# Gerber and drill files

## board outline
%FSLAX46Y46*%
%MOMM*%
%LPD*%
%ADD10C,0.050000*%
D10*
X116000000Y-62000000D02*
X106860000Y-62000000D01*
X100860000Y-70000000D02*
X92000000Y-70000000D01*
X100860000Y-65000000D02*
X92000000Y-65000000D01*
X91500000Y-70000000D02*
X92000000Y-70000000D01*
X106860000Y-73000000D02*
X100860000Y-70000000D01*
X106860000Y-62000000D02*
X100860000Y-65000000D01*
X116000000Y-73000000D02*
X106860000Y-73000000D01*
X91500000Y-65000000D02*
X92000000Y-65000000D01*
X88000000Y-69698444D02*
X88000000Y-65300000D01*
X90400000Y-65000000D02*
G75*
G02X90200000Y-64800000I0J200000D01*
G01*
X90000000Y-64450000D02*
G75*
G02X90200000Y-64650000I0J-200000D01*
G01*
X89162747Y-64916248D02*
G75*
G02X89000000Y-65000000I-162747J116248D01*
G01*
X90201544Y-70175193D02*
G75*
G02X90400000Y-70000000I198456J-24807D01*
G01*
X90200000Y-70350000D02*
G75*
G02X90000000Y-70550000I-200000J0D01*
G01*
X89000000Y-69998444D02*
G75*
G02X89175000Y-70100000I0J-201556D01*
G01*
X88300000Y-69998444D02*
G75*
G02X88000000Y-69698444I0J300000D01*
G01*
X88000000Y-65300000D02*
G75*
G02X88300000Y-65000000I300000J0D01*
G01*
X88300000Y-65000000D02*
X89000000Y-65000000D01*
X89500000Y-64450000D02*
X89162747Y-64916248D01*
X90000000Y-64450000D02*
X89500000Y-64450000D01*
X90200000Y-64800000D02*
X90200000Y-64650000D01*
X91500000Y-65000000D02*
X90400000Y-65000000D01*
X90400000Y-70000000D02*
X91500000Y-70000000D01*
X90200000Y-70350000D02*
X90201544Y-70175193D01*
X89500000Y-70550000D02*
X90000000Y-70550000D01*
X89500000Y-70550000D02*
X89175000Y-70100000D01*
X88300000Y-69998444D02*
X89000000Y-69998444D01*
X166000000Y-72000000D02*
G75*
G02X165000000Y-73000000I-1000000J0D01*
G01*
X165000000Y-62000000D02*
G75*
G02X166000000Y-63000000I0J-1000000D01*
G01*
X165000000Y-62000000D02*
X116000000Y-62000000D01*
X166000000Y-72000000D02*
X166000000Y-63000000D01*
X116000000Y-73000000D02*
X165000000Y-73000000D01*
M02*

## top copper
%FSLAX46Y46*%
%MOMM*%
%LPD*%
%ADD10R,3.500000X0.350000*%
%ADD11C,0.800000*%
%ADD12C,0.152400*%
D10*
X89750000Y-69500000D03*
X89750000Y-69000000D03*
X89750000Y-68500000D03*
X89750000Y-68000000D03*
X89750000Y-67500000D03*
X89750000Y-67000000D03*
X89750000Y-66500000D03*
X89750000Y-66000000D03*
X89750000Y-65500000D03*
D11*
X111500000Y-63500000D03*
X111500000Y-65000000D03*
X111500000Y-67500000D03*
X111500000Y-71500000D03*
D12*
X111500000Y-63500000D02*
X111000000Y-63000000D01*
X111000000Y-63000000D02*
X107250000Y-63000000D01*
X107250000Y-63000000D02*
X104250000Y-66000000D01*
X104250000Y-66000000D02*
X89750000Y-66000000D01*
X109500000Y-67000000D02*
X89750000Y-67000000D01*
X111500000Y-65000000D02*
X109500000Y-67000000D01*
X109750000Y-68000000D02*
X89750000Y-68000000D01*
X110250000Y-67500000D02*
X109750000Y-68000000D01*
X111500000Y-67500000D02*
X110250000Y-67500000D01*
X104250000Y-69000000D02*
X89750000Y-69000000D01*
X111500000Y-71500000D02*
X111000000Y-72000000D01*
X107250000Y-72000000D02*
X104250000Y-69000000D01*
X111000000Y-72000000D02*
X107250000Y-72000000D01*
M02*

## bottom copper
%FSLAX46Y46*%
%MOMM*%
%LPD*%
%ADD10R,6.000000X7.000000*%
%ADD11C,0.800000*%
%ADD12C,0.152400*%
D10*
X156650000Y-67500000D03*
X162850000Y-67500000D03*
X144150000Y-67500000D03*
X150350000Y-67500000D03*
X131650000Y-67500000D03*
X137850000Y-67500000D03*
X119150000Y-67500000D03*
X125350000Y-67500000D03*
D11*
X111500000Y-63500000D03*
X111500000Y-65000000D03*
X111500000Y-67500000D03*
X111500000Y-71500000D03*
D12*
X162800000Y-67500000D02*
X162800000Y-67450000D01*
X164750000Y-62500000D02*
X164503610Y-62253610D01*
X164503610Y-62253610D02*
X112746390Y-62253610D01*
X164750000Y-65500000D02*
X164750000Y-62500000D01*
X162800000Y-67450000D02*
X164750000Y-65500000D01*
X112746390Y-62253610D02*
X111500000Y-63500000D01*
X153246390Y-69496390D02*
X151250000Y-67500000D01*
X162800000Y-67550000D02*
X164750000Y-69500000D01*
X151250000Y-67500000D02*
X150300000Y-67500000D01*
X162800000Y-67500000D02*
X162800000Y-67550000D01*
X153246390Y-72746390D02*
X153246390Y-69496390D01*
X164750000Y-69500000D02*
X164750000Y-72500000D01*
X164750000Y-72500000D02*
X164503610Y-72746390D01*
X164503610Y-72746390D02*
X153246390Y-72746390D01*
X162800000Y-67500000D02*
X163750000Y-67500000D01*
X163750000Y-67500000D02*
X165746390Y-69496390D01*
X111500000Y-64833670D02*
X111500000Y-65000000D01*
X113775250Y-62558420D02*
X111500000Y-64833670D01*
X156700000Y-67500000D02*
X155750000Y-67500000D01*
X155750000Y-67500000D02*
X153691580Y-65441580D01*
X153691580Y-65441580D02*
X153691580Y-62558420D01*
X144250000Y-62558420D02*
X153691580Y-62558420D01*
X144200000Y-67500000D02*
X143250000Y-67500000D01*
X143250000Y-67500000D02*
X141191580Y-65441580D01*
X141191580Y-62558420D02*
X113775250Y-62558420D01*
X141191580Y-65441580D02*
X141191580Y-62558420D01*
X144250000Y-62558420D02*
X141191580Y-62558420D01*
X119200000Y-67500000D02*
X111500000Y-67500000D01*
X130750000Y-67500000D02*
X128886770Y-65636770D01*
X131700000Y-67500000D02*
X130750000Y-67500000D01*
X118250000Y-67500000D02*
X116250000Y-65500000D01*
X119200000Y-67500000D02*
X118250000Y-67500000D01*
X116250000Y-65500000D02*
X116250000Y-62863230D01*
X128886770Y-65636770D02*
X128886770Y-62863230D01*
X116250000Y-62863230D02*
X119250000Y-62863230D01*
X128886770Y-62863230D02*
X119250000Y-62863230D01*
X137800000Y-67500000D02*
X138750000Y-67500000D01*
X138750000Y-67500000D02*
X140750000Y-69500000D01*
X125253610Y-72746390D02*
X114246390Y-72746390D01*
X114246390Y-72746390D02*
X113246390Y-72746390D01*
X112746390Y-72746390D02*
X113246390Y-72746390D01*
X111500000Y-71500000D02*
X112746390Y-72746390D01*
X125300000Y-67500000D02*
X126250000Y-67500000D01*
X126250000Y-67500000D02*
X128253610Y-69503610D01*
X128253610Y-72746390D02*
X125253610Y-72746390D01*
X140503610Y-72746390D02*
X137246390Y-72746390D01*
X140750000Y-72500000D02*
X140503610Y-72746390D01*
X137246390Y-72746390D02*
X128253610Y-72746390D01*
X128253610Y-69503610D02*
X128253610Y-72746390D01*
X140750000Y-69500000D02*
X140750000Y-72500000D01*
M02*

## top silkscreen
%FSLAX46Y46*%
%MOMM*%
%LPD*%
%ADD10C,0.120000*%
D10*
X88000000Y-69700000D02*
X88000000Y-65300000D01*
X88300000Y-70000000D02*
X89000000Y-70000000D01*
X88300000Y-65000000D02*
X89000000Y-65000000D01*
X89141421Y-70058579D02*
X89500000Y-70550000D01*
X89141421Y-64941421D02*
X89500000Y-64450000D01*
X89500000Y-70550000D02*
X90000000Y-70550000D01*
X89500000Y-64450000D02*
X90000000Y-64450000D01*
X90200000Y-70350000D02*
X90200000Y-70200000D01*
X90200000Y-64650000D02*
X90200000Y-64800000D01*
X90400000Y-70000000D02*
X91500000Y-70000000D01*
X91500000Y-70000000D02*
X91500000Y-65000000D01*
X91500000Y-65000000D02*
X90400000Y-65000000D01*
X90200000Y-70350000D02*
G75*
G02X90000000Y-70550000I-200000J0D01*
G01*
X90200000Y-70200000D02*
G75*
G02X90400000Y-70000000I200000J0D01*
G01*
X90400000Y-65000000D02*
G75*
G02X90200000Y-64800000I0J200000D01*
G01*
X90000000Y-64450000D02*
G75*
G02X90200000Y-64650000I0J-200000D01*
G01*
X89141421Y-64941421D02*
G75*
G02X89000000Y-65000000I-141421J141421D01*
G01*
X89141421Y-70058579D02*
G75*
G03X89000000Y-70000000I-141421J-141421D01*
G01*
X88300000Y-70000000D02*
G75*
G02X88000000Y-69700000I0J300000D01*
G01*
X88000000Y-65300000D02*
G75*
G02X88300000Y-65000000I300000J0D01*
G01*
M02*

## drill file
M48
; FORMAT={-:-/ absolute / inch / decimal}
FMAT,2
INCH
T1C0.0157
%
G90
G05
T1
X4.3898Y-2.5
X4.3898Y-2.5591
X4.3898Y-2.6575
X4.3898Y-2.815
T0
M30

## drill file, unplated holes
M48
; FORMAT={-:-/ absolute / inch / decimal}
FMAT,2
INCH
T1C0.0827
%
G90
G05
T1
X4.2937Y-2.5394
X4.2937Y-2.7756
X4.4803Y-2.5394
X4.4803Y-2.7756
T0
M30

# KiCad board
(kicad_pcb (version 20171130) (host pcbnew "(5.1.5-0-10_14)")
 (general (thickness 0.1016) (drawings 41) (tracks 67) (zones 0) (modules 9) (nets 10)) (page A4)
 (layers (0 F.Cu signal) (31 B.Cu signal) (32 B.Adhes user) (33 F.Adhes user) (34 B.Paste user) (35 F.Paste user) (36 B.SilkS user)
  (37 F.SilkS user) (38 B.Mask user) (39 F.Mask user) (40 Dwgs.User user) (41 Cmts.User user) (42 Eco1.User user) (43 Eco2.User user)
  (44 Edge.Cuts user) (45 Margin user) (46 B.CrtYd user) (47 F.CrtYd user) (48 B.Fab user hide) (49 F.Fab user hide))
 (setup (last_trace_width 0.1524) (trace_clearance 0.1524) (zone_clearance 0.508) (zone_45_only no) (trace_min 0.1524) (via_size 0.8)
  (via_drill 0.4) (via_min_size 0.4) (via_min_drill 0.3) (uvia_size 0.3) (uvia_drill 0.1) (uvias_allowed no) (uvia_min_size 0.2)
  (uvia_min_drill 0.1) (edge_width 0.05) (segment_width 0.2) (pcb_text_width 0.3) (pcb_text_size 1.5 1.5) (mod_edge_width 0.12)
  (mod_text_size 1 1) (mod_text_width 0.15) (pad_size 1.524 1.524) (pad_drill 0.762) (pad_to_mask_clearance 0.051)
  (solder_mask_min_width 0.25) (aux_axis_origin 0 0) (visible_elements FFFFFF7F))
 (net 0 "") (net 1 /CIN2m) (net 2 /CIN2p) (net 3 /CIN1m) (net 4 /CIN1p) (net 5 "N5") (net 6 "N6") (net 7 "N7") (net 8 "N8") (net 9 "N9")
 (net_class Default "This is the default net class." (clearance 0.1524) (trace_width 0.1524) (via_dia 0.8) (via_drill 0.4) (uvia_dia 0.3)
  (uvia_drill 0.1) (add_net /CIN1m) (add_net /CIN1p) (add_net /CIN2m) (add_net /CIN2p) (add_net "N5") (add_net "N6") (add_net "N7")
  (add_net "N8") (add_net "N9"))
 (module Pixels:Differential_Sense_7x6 (layer B.Cu) (at 159.75 67.5)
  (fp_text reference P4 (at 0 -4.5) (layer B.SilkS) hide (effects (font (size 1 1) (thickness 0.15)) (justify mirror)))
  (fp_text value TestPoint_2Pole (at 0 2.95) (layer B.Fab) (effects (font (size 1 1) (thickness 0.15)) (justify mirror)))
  (pad 1 smd rect (at -3.1 0) (size 6 7) (layers B.Cu) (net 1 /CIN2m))
  (pad 2 smd rect (at 3.1 0) (size 6 7) (layers B.Cu) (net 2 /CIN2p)))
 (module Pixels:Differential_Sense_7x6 (layer B.Cu) (at 147.25 67.5)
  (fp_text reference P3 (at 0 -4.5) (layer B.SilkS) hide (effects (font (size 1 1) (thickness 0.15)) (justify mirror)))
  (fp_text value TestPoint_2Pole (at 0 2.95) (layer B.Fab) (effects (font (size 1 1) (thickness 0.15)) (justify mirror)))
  (pad 1 smd rect (at -3.1 0) (size 6 7) (layers B.Cu) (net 1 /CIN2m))
  (pad 2 smd rect (at 3.1 0) (size 6 7) (layers B.Cu) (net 2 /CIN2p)))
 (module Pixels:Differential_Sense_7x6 (layer B.Cu) (at 134.75 67.5)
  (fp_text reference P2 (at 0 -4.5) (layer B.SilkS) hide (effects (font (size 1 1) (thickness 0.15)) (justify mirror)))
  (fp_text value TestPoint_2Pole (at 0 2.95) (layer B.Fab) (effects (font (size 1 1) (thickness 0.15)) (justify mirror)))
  (pad 1 smd rect (at -3.1 0) (size 6 7) (layers B.Cu) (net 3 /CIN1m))
  (pad 2 smd rect (at 3.1 0) (size 6 7) (layers B.Cu) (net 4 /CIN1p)))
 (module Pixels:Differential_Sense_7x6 (layer B.Cu) (at 122.25 67.5)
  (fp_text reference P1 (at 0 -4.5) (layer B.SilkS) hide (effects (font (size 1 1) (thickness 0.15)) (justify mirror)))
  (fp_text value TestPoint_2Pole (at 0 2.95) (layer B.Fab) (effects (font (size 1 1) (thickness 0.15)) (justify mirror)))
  (pad 1 smd rect (at -3.1 0) (size 6 7) (layers B.Cu) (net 3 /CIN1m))
  (pad 2 smd rect (at 3.1 0) (size 6 7) (layers B.Cu) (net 4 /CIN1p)))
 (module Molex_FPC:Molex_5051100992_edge (layer F.Cu) (at 91.5 67.5 90)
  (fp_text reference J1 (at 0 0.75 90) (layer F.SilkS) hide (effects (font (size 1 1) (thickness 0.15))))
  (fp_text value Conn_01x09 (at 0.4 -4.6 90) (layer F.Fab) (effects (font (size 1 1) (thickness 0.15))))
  (fp_line (start -2.2 -3.5) (end 2.2 -3.5) (layer F.SilkS) (width 0.12))
  (fp_line (start -2.5 -3.2) (end -2.5 -2.5) (layer F.SilkS) (width 0.12))
  (fp_line (start 2.5 -3.2) (end 2.5 -2.5) (layer F.SilkS) (width 0.12))
  (fp_line (start -2.558579 -2.358579) (end -3.05 -2) (layer F.SilkS) (width 0.12))
  (fp_line (start 2.558579 -2.358579) (end 3.05 -2) (layer F.SilkS) (width 0.12))
  (fp_line (start -3.05 -2) (end -3.05 -1.5) (layer F.SilkS) (width 0.12))
  (fp_line (start 3.05 -2) (end 3.05 -1.5) (layer F.SilkS) (width 0.12))
  (fp_line (start -2.85 -1.3) (end -2.7 -1.3) (layer F.SilkS) (width 0.12))
  (fp_line (start 2.85 -1.3) (end 2.7 -1.3) (layer F.SilkS) (width 0.12))
  (fp_line (start -2.5 -1.1) (end -2.5 0) (layer F.SilkS) (width 0.12))
  (fp_line (start -2.5 0) (end 2.5 0) (layer F.SilkS) (width 0.12))
  (fp_line (start 2.5 0) (end 2.5 -1.1) (layer F.SilkS) (width 0.12))
  (fp_arc (start -2.85 -1.5) (end -3.05 -1.5) (angle -90) (layer F.SilkS) (width 0.12))
  (fp_arc (start -2.7 -1.1) (end -2.5 -1.1) (angle -90) (layer F.SilkS) (width 0.12))
  (fp_arc (start 2.7 -1.1) (end 2.7 -1.3) (angle -90) (layer F.SilkS) (width 0.12))
  (fp_arc (start 2.85 -1.5) (end 2.85 -1.3) (angle -90) (layer F.SilkS) (width 0.12))
  (fp_arc (start 2.7 -2.5) (end 2.5 -2.5) (angle -45) (layer F.SilkS) (width 0.12))
  (fp_arc (start -2.7 -2.5) (end -2.5 -2.5) (angle 45) (layer F.SilkS) (width 0.12))
  (fp_arc (start -2.2 -3.2) (end -2.2 -3.5) (angle -90) (layer F.SilkS) (width 0.12))
  (fp_arc (start 2.2 -3.2) (end 2.5 -3.2) (angle -90) (layer F.SilkS) (width 0.12))
  (pad 1 connect rect (at -2 -1.75 90) (size 0.35 3.5) (layers F.Cu F.Mask) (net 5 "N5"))
  (pad 2 connect rect (at -1.5 -1.75 90) (size 0.35 3.5) (layers F.Cu F.Mask) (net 4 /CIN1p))
  (pad 3 connect rect (at -1 -1.75 90) (size 0.35 3.5) (layers F.Cu F.Mask) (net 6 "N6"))
  (pad 4 connect rect (at -0.5 -1.75 90) (size 0.35 3.5) (layers F.Cu F.Mask) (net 3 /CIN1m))
  (pad 5 connect rect (at 0 -1.75 90) (size 0.35 3.5) (layers F.Cu F.Mask) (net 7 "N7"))
  (pad 6 connect rect (at 0.5 -1.75 90) (size 0.35 3.5) (layers F.Cu F.Mask) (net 1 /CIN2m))
  (pad 7 connect rect (at 1 -1.75 90) (size 0.35 3.5) (layers F.Cu F.Mask) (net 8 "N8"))
  (pad 8 connect rect (at 1.5 -1.75 90) (size 0.35 3.5) (layers F.Cu F.Mask) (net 2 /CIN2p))
  (pad 9 connect rect (at 2 -1.75 90) (size 0.35 3.5) (layers F.Cu F.Mask) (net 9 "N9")))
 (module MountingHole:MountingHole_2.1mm (layer F.Cu) (at 109.06 64.5)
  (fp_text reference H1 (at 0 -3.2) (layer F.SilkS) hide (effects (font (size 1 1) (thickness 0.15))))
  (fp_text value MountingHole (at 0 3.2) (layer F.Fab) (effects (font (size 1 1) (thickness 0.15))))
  (pad "" np_thru_hole circle (at 0 0) (size 2.1 2.1) (drill 2.1) (layers *.Cu *.Mask)))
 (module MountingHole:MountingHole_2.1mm (layer F.Cu) (at 109.06 70.5)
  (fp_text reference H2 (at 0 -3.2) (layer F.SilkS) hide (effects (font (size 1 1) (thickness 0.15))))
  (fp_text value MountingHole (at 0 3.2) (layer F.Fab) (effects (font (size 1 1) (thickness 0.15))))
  (pad "" np_thru_hole circle (at 0 0) (size 2.1 2.1) (drill 2.1) (layers *.Cu *.Mask)))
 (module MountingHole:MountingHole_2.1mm (layer F.Cu) (at 113.8 64.5)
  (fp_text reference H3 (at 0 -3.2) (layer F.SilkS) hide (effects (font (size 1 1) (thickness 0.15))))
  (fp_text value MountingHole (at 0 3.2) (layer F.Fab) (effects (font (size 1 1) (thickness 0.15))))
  (pad "" np_thru_hole circle (at 0 0) (size 2.1 2.1) (drill 2.1) (layers *.Cu *.Mask)))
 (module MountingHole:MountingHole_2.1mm (layer F.Cu) (at 113.8 70.5)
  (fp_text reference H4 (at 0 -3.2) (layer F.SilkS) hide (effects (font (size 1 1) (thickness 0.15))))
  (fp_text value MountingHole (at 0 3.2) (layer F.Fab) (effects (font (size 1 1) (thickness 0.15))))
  (pad "" np_thru_hole circle (at 0 0) (size 2.1 2.1) (drill 2.1) (layers *.Cu *.Mask)))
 (gr_line (start 116 62) (end 106.86 62) (layer Edge.Cuts) (width 0.05))
 (gr_line (start 100.86 70) (end 92 70) (layer Edge.Cuts) (width 0.05))
 (gr_line (start 100.86 65) (end 92 65) (layer Edge.Cuts) (width 0.05))
 (gr_line (start 91.5 70) (end 92 70) (layer Edge.Cuts) (width 0.05))
 (gr_line (start 106.86 73) (end 100.86 70) (layer Edge.Cuts) (width 0.05))
 (gr_line (start 106.86 62) (end 100.86 65) (layer Edge.Cuts) (width 0.05))
 (gr_line (start 116 73) (end 106.86 73) (layer Edge.Cuts) (width 0.05))
 (gr_line (start 91.5 65) (end 92 65) (layer Edge.Cuts) (width 0.05))
 (gr_line (start 88 69.698444) (end 88 65.3) (layer Edge.Cuts) (width 0.05))
 (gr_arc (start 90.4 64.8) (end 90.2 64.8) (angle -90) (layer Edge.Cuts) (width 0.05))
 (gr_arc (start 90 64.65) (end 90.2 64.65) (angle -90) (layer Edge.Cuts) (width 0.05))
 (gr_arc (start 89 64.8) (end 89 65) (angle -54.46228891) (layer Edge.Cuts) (width 0.05))
 (gr_arc (start 90.4 70.2) (end 90.4 70) (angle -82.87498365) (layer Edge.Cuts) (width 0.05))
 (gr_arc (start 90 70.35) (end 90 70.55) (angle -90) (layer Edge.Cuts) (width 0.05))
 (gr_arc (start 89 70.2) (end 89.175 70.1) (angle -60.2551187) (layer Edge.Cuts) (width 0.05))
 (gr_arc (start 88.3 69.698444) (end 88 69.698444) (angle -90) (layer Edge.Cuts) (width 0.05))
 (gr_arc (start 88.3 65.3) (end 88.3 65) (angle -90) (layer Edge.Cuts) (width 0.05))
 (gr_line (start 88.3 65) (end 89 65) (layer Edge.Cuts) (width 0.05))
 (gr_line (start 89.5 64.45) (end 89.162747 64.916248) (layer Edge.Cuts) (width 0.05))
 (gr_line (start 90 64.45) (end 89.5 64.45) (layer Edge.Cuts) (width 0.05))
 (gr_line (start 90.2 64.8) (end 90.2 64.65) (layer Edge.Cuts) (width 0.05))
 (gr_line (start 91.5 65) (end 90.4 65) (layer Edge.Cuts) (width 0.05))
 (gr_line (start 90.4 70) (end 91.5 70) (layer Edge.Cuts) (width 0.05))
 (gr_line (start 90.2 70.35) (end 90.201544 70.175193) (layer Edge.Cuts) (width 0.05))
 (gr_line (start 89.5 70.55) (end 90 70.55) (layer Edge.Cuts) (width 0.05))
 (gr_line (start 89.5 70.55) (end 89.175 70.1) (layer Edge.Cuts) (width 0.05))
 (gr_line (start 88.3 69.998444) (end 89 69.998444) (layer Edge.Cuts) (width 0.05))
 (gr_arc (start 165 72) (end 165 73) (angle -90) (layer Edge.Cuts) (width 0.05))
 (gr_arc (start 165 63) (end 166 63) (angle -90) (layer Edge.Cuts) (width 0.05))
 (gr_line (start 165 62) (end 116 62) (layer Edge.Cuts) (width 0.05))
 (gr_line (start 166 72) (end 166 63) (layer Edge.Cuts) (width 0.05))
 (gr_line (start 116 73) (end 165 73) (layer Edge.Cuts) (width 0.05))
 (via (at 111.5 63.5) (size 0.8) (drill 0.4) (layers F.Cu B.Cu) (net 2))
 (segment (start 162.8 67.5) (end 162.8 67.45) (width 0.1524) (layer B.Cu) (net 2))
 (segment (start 164.75 62.5) (end 164.50361 62.25361) (width 0.1524) (layer B.Cu) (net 2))
 (segment (start 164.50361 62.25361) (end 112.74639 62.25361) (width 0.1524) (layer B.Cu) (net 2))
 (segment (start 164.75 65.5) (end 164.75 62.5) (width 0.1524) (layer B.Cu) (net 2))
 (segment (start 162.8 67.45) (end 164.75 65.5) (width 0.1524) (layer B.Cu) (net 2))
 (segment (start 112.74639 62.25361) (end 111.5 63.5) (width 0.1524) (layer B.Cu) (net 2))
 (segment (start 111.5 63.5) (end 111 63) (width 0.1524) (layer F.Cu) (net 2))
 (segment (start 111 63) (end 107.25 63) (width 0.1524) (layer F.Cu) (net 2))
 (segment (start 107.25 63) (end 104.25 66) (width 0.1524) (layer F.Cu) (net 2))
 (segment (start 104.25 66) (end 89.75 66) (width 0.1524) (layer F.Cu) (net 2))
 (segment (start 153.24639 69.49639) (end 151.25 67.5) (width 0.1524) (layer B.Cu) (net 2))
 (segment (start 162.8 67.55) (end 164.75 69.5) (width 0.1524) (layer B.Cu) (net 2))
 (segment (start 151.25 67.5) (end 150.3 67.5) (width 0.1524) (layer B.Cu) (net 2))
 (segment (start 162.8 67.5) (end 162.8 67.55) (width 0.1524) (layer B.Cu) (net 2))
 (segment (start 153.24639 72.74639) (end 153.24639 69.49639) (width 0.1524) (layer B.Cu) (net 2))
 (segment (start 164.75 69.5) (end 164.75 72.5) (width 0.1524) (layer B.Cu) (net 2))
 (segment (start 164.75 72.5) (end 164.50361 72.74639) (width 0.1524) (layer B.Cu) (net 2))
 (segment (start 164.50361 72.74639) (end 153.24639 72.74639) (width 0.1524) (layer B.Cu) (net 2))
 (segment (start 162.8 67.5) (end 163.75 67.5) (width 0.1524) (layer B.Cu) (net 2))
 (segment (start 163.75 67.5) (end 165.74639 69.49639) (width 0.1524) (layer B.Cu) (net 2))
 (segment (start 109.5 67) (end 89.75 67) (width 0.1524) (layer F.Cu) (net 1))
 (segment (start 111.5 64.83367) (end 111.5 65) (width 0.1524) (layer B.Cu) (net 1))
 (via (at 111.5 65) (size 0.8) (drill 0.4) (layers F.Cu B.Cu) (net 1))
 (segment (start 111.5 65) (end 109.5 67) (width 0.1524) (layer F.Cu) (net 1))
 (segment (start 113.77525 62.55842) (end 111.5 64.83367) (width 0.1524) (layer B.Cu) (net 1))
 (segment (start 156.7 67.5) (end 155.75 67.5) (width 0.1524) (layer B.Cu) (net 1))
 (segment (start 155.75 67.5) (end 153.69158 65.44158) (width 0.1524) (layer B.Cu) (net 1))
 (segment (start 153.69158 65.44158) (end 153.69158 62.55842) (width 0.1524) (layer B.Cu) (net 1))
 (segment (start 144.25 62.55842) (end 153.69158 62.55842) (width 0.1524) (layer B.Cu) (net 1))
 (segment (start 144.2 67.5) (end 143.25 67.5) (width 0.1524) (layer B.Cu) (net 1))
 (segment (start 143.25 67.5) (end 141.19158 65.44158) (width 0.1524) (layer B.Cu) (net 1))
 (segment (start 141.19158 62.55842) (end 113.77525 62.55842) (width 0.1524) (layer B.Cu) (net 1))
 (segment (start 141.19158 65.44158) (end 141.19158 62.55842) (width 0.1524) (layer B.Cu) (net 1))
 (segment (start 144.25 62.55842) (end 141.19158 62.55842) (width 0.1524) (layer B.Cu) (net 1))
 (via (at 111.5 67.5) (size 0.8) (drill 0.4) (layers F.Cu B.Cu) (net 3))
 (segment (start 119.2 67.5) (end 111.5 67.5) (width 0.1524) (layer B.Cu) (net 3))
 (segment (start 109.75 68) (end 89.75 68) (width 0.1524) (layer F.Cu) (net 3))
 (segment (start 110.25 67.5) (end 109.75 68) (width 0.1524) (layer F.Cu) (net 3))
 (segment (start 111.5 67.5) (end 110.25 67.5) (width 0.1524) (layer F.Cu) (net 3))
 (segment (start 130.75 67.5) (end 128.88677 65.63677) (width 0.1524) (layer B.Cu) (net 3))
 (segment (start 131.7 67.5) (end 130.75 67.5) (width 0.1524) (layer B.Cu) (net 3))
 (segment (start 118.25 67.5) (end 116.25 65.5) (width 0.1524) (layer B.Cu) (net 3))
 (segment (start 119.2 67.5) (end 118.25 67.5) (width 0.1524) (layer B.Cu) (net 3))
 (segment (start 116.25 65.5) (end 116.25 62.86323) (width 0.1524) (layer B.Cu) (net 3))
 (segment (start 128.88677 65.63677) (end 128.88677 62.86323) (width 0.1524) (layer B.Cu) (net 3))
 (segment (start 116.25 62.86323) (end 119.25 62.86323) (width 0.1524) (layer B.Cu) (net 3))
 (segment (start 128.88677 62.86323) (end 119.25 62.86323) (width 0.1524) (layer B.Cu) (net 3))
 (via (at 111.5 71.5) (size 0.8) (drill 0.4) (layers F.Cu B.Cu) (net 4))
 (segment (start 104.25 69) (end 89.75 69) (width 0.1524) (layer F.Cu) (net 4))
 (segment (start 111.5 71.5) (end 111 72) (width 0.1524) (layer F.Cu) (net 4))
 (segment (start 107.25 72) (end 104.25 69) (width 0.1524) (layer F.Cu) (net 4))
 (segment (start 111 72) (end 107.25 72) (width 0.1524) (layer F.Cu) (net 4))
 (segment (start 137.8 67.5) (end 138.75 67.5) (width 0.1524) (layer B.Cu) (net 4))
 (segment (start 138.75 67.5) (end 140.75 69.5) (width 0.1524) (layer B.Cu) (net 4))
 (segment (start 125.25361 72.74639) (end 114.24639 72.74639) (width 0.1524) (layer B.Cu) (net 4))
 (segment (start 114.24639 72.74639) (end 113.24639 72.74639) (width 0.1524) (layer B.Cu) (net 4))
 (segment (start 112.74639 72.74639) (end 113.24639 72.74639) (width 0.1524) (layer B.Cu) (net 4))
 (segment (start 111.5 71.5) (end 112.74639 72.74639) (width 0.1524) (layer B.Cu) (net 4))
 (segment (start 125.3 67.5) (end 126.25 67.5) (width 0.1524) (layer B.Cu) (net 4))
 (segment (start 126.25 67.5) (end 128.25361 69.50361) (width 0.1524) (layer B.Cu) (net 4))
 (segment (start 128.25361 72.74639) (end 125.25361 72.74639) (width 0.1524) (layer B.Cu) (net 4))
 (segment (start 140.50361 72.74639) (end 137.24639 72.74639) (width 0.1524) (layer B.Cu) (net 4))
 (segment (start 140.75 72.5) (end 140.50361 72.74639) (width 0.1524) (layer B.Cu) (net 4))
 (segment (start 137.24639 72.74639) (end 128.25361 72.74639) (width 0.1524) (layer B.Cu) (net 4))
 (segment (start 128.25361 69.50361) (end 128.25361 72.74639) (width 0.1524) (layer B.Cu) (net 4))
 (segment (start 140.75 69.5) (end 140.75 72.5) (width 0.1524) (layer B.Cu) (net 4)))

